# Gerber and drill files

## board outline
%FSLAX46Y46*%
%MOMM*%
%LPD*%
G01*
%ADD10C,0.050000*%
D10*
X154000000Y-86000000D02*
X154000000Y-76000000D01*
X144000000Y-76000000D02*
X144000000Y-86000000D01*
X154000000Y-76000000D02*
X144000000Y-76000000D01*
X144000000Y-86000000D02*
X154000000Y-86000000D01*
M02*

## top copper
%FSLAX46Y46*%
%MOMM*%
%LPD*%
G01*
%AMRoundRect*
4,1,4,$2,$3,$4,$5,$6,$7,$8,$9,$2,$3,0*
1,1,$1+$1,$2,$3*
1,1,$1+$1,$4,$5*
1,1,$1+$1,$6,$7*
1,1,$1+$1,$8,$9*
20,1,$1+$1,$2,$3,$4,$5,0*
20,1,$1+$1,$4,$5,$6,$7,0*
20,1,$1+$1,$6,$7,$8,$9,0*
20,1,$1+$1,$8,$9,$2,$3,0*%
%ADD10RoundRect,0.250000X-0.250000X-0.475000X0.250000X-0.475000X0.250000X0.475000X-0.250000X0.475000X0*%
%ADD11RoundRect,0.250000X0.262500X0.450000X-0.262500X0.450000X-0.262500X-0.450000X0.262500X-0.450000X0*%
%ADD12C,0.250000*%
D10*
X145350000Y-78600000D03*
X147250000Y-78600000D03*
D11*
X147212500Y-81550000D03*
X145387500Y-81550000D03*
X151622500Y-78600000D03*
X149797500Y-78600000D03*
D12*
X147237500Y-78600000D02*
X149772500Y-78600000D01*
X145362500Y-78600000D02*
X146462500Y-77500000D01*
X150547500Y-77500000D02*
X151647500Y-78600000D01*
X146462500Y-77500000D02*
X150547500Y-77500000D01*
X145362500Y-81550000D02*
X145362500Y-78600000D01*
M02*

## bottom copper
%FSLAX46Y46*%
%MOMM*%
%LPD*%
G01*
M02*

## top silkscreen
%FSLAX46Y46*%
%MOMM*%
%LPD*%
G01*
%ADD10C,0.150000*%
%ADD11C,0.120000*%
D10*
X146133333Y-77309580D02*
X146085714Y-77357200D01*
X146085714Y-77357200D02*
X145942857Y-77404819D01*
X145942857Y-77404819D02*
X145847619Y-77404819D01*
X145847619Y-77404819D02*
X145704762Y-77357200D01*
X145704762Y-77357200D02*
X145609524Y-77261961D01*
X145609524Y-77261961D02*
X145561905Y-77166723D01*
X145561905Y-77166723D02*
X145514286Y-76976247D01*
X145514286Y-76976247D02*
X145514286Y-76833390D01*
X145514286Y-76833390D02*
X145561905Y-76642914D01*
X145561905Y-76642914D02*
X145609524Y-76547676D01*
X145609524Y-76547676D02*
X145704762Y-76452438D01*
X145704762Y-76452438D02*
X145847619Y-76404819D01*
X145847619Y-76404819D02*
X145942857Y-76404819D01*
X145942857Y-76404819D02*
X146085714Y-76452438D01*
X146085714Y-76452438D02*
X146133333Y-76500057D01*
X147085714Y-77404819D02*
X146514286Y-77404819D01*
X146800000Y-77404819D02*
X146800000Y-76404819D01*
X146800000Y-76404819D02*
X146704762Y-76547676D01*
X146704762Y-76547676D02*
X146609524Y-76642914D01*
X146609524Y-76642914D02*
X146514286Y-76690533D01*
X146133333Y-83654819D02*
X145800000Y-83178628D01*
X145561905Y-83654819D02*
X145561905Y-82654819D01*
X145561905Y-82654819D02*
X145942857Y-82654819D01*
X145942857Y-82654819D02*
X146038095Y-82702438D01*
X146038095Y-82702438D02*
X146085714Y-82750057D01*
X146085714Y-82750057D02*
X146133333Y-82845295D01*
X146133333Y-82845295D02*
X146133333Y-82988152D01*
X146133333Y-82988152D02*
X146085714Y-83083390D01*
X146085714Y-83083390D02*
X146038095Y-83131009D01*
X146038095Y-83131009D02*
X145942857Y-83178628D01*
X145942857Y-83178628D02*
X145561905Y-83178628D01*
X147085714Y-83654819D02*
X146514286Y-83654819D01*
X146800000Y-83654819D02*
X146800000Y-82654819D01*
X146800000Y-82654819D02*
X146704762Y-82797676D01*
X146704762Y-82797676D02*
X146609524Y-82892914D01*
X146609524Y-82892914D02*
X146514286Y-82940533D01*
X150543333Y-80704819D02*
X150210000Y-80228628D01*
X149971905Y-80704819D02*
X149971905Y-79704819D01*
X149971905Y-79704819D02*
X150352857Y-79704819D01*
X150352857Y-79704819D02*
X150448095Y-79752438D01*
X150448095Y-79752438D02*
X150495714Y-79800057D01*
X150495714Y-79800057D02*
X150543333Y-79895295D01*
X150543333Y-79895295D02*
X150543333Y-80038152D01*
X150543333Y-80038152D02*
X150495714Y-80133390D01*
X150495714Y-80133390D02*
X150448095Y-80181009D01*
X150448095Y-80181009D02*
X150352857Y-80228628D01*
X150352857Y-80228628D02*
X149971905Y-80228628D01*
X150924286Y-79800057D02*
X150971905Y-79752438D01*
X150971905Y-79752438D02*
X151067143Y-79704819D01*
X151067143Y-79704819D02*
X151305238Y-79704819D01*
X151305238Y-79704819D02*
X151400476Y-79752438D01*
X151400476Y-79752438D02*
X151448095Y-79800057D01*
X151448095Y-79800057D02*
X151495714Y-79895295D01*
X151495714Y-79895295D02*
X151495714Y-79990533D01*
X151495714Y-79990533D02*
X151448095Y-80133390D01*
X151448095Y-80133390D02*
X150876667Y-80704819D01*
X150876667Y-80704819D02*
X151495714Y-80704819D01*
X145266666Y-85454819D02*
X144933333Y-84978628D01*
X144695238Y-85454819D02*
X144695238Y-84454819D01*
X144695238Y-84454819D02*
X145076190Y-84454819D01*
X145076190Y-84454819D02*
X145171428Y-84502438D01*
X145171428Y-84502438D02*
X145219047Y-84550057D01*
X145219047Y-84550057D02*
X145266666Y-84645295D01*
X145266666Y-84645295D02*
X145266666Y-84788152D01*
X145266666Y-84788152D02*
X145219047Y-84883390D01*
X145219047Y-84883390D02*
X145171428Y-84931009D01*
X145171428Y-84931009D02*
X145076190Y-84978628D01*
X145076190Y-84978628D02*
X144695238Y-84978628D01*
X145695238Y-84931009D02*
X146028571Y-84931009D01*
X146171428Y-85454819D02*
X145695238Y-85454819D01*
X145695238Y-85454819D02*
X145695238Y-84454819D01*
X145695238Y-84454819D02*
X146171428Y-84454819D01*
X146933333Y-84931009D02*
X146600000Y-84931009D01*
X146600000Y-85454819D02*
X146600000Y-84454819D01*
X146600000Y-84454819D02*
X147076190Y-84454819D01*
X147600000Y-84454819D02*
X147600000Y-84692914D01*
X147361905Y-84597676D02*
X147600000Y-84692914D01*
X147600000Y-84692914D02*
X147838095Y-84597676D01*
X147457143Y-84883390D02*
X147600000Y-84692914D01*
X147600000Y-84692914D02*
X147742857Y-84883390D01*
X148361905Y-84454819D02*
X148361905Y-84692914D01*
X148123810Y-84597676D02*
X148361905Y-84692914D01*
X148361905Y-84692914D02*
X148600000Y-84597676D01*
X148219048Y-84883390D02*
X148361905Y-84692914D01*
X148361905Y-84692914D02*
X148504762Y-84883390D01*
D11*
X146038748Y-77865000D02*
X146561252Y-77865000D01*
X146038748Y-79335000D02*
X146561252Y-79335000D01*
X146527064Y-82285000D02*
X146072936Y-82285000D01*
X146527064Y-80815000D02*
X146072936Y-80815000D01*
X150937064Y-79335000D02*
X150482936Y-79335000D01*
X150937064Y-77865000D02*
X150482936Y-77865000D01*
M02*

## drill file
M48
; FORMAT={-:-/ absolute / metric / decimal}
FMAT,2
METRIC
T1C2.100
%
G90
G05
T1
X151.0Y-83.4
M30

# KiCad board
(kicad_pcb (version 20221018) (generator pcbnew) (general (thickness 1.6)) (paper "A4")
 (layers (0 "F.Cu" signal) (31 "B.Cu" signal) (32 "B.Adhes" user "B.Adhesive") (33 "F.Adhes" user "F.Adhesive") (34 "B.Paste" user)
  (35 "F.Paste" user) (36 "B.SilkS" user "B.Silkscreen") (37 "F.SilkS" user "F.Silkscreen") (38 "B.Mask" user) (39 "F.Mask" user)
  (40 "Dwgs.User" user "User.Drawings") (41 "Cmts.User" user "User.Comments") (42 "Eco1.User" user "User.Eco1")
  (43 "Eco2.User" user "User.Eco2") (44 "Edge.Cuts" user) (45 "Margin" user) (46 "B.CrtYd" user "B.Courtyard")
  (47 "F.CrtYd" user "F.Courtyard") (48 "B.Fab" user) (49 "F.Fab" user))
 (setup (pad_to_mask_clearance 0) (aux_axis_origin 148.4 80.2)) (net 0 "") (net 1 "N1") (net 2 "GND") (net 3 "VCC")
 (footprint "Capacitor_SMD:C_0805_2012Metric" (layer "F.Cu") (at 146.3 78.6)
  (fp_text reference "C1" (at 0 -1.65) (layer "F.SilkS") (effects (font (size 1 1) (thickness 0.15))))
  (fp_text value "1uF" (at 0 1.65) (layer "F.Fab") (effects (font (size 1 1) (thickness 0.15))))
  (fp_line (start -0.261252 -0.735) (end 0.261252 -0.735) (stroke (width 0.12) (type solid)) (layer "F.SilkS"))
  (fp_line (start -0.261252 0.735) (end 0.261252 0.735) (stroke (width 0.12) (type solid)) (layer "F.SilkS"))
  (pad "1" smd roundrect (at -0.95 0) (size 1 1.45) (layers "F.Cu" "F.Paste" "F.Mask") (roundrect_rratio 0.25) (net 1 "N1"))
  (pad "2" smd roundrect (at 0.95 0) (size 1 1.45) (layers "F.Cu" "F.Paste" "F.Mask") (roundrect_rratio 0.25) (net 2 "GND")))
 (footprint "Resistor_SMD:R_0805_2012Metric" (layer "F.Cu") (at 146.3 81.55 180)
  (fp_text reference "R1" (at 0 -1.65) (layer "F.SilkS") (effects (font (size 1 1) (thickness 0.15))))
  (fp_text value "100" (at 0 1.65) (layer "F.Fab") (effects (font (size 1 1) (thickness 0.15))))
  (fp_line (start -0.227064 -0.735) (end 0.227064 -0.735) (stroke (width 0.12) (type solid)) (layer "F.SilkS"))
  (fp_line (start -0.227064 0.735) (end 0.227064 0.735) (stroke (width 0.12) (type solid)) (layer "F.SilkS"))
  (pad "1" smd roundrect (at -0.9125 0 180) (size 1.025 1.4) (layers "F.Cu" "F.Paste" "F.Mask") (roundrect_rratio 0.243902) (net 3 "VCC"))
  (pad "2" smd roundrect (at 0.9125 0 180) (size 1.025 1.4) (layers "F.Cu" "F.Paste" "F.Mask") (roundrect_rratio 0.243902) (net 1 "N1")))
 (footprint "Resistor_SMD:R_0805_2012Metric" (layer "F.Cu") (at 150.71 78.6 180)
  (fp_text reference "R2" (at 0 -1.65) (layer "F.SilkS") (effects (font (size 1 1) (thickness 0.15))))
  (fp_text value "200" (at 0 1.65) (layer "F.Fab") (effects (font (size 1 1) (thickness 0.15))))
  (fp_line (start -0.227064 -0.735) (end 0.227064 -0.735) (stroke (width 0.12) (type solid)) (layer "F.SilkS"))
  (fp_line (start -0.227064 0.735) (end 0.227064 0.735) (stroke (width 0.12) (type solid)) (layer "F.SilkS"))
  (pad "1" smd roundrect (at -0.9125 0 180) (size 1.025 1.4) (layers "F.Cu" "F.Paste" "F.Mask") (roundrect_rratio 0.243902) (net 1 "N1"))
  (pad "2" smd roundrect (at 0.9125 0 180) (size 1.025 1.4) (layers "F.Cu" "F.Paste" "F.Mask") (roundrect_rratio 0.243902) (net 2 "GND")))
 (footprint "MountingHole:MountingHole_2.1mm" (layer "F.Cu") (at 151 83.4)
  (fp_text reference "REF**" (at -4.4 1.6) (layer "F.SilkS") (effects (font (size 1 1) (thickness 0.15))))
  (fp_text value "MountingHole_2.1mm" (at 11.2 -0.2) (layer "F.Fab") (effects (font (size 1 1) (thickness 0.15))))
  (pad "" np_thru_hole circle (at 0 0) (size 2.1 2.1) (drill 2.1) (layers "*.Cu" "*.Mask")))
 (gr_line (start 154 86) (end 154 76) (stroke (width 0.05) (type solid)) (layer "Edge.Cuts"))
 (gr_line (start 144 76) (end 144 86) (stroke (width 0.05) (type solid)) (layer "Edge.Cuts"))
 (gr_line (start 154 76) (end 144 76) (stroke (width 0.05) (type solid)) (layer "Edge.Cuts"))
 (gr_line (start 144 86) (end 154 86) (stroke (width 0.05) (type solid)) (layer "Edge.Cuts"))
 (segment (start 147.2375 78.6) (end 149.7725 78.6) (width 0.25) (layer "F.Cu") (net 2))
 (segment (start 145.3625 78.6) (end 146.4625 77.5) (width 0.25) (layer "F.Cu") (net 1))
 (segment (start 150.5475 77.5) (end 151.6475 78.6) (width 0.25) (layer "F.Cu") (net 1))
 (segment (start 146.4625 77.5) (end 150.5475 77.5) (width 0.25) (layer "F.Cu") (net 1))
 (segment (start 145.3625 81.55) (end 145.3625 78.6) (width 0.25) (layer "F.Cu") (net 1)))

